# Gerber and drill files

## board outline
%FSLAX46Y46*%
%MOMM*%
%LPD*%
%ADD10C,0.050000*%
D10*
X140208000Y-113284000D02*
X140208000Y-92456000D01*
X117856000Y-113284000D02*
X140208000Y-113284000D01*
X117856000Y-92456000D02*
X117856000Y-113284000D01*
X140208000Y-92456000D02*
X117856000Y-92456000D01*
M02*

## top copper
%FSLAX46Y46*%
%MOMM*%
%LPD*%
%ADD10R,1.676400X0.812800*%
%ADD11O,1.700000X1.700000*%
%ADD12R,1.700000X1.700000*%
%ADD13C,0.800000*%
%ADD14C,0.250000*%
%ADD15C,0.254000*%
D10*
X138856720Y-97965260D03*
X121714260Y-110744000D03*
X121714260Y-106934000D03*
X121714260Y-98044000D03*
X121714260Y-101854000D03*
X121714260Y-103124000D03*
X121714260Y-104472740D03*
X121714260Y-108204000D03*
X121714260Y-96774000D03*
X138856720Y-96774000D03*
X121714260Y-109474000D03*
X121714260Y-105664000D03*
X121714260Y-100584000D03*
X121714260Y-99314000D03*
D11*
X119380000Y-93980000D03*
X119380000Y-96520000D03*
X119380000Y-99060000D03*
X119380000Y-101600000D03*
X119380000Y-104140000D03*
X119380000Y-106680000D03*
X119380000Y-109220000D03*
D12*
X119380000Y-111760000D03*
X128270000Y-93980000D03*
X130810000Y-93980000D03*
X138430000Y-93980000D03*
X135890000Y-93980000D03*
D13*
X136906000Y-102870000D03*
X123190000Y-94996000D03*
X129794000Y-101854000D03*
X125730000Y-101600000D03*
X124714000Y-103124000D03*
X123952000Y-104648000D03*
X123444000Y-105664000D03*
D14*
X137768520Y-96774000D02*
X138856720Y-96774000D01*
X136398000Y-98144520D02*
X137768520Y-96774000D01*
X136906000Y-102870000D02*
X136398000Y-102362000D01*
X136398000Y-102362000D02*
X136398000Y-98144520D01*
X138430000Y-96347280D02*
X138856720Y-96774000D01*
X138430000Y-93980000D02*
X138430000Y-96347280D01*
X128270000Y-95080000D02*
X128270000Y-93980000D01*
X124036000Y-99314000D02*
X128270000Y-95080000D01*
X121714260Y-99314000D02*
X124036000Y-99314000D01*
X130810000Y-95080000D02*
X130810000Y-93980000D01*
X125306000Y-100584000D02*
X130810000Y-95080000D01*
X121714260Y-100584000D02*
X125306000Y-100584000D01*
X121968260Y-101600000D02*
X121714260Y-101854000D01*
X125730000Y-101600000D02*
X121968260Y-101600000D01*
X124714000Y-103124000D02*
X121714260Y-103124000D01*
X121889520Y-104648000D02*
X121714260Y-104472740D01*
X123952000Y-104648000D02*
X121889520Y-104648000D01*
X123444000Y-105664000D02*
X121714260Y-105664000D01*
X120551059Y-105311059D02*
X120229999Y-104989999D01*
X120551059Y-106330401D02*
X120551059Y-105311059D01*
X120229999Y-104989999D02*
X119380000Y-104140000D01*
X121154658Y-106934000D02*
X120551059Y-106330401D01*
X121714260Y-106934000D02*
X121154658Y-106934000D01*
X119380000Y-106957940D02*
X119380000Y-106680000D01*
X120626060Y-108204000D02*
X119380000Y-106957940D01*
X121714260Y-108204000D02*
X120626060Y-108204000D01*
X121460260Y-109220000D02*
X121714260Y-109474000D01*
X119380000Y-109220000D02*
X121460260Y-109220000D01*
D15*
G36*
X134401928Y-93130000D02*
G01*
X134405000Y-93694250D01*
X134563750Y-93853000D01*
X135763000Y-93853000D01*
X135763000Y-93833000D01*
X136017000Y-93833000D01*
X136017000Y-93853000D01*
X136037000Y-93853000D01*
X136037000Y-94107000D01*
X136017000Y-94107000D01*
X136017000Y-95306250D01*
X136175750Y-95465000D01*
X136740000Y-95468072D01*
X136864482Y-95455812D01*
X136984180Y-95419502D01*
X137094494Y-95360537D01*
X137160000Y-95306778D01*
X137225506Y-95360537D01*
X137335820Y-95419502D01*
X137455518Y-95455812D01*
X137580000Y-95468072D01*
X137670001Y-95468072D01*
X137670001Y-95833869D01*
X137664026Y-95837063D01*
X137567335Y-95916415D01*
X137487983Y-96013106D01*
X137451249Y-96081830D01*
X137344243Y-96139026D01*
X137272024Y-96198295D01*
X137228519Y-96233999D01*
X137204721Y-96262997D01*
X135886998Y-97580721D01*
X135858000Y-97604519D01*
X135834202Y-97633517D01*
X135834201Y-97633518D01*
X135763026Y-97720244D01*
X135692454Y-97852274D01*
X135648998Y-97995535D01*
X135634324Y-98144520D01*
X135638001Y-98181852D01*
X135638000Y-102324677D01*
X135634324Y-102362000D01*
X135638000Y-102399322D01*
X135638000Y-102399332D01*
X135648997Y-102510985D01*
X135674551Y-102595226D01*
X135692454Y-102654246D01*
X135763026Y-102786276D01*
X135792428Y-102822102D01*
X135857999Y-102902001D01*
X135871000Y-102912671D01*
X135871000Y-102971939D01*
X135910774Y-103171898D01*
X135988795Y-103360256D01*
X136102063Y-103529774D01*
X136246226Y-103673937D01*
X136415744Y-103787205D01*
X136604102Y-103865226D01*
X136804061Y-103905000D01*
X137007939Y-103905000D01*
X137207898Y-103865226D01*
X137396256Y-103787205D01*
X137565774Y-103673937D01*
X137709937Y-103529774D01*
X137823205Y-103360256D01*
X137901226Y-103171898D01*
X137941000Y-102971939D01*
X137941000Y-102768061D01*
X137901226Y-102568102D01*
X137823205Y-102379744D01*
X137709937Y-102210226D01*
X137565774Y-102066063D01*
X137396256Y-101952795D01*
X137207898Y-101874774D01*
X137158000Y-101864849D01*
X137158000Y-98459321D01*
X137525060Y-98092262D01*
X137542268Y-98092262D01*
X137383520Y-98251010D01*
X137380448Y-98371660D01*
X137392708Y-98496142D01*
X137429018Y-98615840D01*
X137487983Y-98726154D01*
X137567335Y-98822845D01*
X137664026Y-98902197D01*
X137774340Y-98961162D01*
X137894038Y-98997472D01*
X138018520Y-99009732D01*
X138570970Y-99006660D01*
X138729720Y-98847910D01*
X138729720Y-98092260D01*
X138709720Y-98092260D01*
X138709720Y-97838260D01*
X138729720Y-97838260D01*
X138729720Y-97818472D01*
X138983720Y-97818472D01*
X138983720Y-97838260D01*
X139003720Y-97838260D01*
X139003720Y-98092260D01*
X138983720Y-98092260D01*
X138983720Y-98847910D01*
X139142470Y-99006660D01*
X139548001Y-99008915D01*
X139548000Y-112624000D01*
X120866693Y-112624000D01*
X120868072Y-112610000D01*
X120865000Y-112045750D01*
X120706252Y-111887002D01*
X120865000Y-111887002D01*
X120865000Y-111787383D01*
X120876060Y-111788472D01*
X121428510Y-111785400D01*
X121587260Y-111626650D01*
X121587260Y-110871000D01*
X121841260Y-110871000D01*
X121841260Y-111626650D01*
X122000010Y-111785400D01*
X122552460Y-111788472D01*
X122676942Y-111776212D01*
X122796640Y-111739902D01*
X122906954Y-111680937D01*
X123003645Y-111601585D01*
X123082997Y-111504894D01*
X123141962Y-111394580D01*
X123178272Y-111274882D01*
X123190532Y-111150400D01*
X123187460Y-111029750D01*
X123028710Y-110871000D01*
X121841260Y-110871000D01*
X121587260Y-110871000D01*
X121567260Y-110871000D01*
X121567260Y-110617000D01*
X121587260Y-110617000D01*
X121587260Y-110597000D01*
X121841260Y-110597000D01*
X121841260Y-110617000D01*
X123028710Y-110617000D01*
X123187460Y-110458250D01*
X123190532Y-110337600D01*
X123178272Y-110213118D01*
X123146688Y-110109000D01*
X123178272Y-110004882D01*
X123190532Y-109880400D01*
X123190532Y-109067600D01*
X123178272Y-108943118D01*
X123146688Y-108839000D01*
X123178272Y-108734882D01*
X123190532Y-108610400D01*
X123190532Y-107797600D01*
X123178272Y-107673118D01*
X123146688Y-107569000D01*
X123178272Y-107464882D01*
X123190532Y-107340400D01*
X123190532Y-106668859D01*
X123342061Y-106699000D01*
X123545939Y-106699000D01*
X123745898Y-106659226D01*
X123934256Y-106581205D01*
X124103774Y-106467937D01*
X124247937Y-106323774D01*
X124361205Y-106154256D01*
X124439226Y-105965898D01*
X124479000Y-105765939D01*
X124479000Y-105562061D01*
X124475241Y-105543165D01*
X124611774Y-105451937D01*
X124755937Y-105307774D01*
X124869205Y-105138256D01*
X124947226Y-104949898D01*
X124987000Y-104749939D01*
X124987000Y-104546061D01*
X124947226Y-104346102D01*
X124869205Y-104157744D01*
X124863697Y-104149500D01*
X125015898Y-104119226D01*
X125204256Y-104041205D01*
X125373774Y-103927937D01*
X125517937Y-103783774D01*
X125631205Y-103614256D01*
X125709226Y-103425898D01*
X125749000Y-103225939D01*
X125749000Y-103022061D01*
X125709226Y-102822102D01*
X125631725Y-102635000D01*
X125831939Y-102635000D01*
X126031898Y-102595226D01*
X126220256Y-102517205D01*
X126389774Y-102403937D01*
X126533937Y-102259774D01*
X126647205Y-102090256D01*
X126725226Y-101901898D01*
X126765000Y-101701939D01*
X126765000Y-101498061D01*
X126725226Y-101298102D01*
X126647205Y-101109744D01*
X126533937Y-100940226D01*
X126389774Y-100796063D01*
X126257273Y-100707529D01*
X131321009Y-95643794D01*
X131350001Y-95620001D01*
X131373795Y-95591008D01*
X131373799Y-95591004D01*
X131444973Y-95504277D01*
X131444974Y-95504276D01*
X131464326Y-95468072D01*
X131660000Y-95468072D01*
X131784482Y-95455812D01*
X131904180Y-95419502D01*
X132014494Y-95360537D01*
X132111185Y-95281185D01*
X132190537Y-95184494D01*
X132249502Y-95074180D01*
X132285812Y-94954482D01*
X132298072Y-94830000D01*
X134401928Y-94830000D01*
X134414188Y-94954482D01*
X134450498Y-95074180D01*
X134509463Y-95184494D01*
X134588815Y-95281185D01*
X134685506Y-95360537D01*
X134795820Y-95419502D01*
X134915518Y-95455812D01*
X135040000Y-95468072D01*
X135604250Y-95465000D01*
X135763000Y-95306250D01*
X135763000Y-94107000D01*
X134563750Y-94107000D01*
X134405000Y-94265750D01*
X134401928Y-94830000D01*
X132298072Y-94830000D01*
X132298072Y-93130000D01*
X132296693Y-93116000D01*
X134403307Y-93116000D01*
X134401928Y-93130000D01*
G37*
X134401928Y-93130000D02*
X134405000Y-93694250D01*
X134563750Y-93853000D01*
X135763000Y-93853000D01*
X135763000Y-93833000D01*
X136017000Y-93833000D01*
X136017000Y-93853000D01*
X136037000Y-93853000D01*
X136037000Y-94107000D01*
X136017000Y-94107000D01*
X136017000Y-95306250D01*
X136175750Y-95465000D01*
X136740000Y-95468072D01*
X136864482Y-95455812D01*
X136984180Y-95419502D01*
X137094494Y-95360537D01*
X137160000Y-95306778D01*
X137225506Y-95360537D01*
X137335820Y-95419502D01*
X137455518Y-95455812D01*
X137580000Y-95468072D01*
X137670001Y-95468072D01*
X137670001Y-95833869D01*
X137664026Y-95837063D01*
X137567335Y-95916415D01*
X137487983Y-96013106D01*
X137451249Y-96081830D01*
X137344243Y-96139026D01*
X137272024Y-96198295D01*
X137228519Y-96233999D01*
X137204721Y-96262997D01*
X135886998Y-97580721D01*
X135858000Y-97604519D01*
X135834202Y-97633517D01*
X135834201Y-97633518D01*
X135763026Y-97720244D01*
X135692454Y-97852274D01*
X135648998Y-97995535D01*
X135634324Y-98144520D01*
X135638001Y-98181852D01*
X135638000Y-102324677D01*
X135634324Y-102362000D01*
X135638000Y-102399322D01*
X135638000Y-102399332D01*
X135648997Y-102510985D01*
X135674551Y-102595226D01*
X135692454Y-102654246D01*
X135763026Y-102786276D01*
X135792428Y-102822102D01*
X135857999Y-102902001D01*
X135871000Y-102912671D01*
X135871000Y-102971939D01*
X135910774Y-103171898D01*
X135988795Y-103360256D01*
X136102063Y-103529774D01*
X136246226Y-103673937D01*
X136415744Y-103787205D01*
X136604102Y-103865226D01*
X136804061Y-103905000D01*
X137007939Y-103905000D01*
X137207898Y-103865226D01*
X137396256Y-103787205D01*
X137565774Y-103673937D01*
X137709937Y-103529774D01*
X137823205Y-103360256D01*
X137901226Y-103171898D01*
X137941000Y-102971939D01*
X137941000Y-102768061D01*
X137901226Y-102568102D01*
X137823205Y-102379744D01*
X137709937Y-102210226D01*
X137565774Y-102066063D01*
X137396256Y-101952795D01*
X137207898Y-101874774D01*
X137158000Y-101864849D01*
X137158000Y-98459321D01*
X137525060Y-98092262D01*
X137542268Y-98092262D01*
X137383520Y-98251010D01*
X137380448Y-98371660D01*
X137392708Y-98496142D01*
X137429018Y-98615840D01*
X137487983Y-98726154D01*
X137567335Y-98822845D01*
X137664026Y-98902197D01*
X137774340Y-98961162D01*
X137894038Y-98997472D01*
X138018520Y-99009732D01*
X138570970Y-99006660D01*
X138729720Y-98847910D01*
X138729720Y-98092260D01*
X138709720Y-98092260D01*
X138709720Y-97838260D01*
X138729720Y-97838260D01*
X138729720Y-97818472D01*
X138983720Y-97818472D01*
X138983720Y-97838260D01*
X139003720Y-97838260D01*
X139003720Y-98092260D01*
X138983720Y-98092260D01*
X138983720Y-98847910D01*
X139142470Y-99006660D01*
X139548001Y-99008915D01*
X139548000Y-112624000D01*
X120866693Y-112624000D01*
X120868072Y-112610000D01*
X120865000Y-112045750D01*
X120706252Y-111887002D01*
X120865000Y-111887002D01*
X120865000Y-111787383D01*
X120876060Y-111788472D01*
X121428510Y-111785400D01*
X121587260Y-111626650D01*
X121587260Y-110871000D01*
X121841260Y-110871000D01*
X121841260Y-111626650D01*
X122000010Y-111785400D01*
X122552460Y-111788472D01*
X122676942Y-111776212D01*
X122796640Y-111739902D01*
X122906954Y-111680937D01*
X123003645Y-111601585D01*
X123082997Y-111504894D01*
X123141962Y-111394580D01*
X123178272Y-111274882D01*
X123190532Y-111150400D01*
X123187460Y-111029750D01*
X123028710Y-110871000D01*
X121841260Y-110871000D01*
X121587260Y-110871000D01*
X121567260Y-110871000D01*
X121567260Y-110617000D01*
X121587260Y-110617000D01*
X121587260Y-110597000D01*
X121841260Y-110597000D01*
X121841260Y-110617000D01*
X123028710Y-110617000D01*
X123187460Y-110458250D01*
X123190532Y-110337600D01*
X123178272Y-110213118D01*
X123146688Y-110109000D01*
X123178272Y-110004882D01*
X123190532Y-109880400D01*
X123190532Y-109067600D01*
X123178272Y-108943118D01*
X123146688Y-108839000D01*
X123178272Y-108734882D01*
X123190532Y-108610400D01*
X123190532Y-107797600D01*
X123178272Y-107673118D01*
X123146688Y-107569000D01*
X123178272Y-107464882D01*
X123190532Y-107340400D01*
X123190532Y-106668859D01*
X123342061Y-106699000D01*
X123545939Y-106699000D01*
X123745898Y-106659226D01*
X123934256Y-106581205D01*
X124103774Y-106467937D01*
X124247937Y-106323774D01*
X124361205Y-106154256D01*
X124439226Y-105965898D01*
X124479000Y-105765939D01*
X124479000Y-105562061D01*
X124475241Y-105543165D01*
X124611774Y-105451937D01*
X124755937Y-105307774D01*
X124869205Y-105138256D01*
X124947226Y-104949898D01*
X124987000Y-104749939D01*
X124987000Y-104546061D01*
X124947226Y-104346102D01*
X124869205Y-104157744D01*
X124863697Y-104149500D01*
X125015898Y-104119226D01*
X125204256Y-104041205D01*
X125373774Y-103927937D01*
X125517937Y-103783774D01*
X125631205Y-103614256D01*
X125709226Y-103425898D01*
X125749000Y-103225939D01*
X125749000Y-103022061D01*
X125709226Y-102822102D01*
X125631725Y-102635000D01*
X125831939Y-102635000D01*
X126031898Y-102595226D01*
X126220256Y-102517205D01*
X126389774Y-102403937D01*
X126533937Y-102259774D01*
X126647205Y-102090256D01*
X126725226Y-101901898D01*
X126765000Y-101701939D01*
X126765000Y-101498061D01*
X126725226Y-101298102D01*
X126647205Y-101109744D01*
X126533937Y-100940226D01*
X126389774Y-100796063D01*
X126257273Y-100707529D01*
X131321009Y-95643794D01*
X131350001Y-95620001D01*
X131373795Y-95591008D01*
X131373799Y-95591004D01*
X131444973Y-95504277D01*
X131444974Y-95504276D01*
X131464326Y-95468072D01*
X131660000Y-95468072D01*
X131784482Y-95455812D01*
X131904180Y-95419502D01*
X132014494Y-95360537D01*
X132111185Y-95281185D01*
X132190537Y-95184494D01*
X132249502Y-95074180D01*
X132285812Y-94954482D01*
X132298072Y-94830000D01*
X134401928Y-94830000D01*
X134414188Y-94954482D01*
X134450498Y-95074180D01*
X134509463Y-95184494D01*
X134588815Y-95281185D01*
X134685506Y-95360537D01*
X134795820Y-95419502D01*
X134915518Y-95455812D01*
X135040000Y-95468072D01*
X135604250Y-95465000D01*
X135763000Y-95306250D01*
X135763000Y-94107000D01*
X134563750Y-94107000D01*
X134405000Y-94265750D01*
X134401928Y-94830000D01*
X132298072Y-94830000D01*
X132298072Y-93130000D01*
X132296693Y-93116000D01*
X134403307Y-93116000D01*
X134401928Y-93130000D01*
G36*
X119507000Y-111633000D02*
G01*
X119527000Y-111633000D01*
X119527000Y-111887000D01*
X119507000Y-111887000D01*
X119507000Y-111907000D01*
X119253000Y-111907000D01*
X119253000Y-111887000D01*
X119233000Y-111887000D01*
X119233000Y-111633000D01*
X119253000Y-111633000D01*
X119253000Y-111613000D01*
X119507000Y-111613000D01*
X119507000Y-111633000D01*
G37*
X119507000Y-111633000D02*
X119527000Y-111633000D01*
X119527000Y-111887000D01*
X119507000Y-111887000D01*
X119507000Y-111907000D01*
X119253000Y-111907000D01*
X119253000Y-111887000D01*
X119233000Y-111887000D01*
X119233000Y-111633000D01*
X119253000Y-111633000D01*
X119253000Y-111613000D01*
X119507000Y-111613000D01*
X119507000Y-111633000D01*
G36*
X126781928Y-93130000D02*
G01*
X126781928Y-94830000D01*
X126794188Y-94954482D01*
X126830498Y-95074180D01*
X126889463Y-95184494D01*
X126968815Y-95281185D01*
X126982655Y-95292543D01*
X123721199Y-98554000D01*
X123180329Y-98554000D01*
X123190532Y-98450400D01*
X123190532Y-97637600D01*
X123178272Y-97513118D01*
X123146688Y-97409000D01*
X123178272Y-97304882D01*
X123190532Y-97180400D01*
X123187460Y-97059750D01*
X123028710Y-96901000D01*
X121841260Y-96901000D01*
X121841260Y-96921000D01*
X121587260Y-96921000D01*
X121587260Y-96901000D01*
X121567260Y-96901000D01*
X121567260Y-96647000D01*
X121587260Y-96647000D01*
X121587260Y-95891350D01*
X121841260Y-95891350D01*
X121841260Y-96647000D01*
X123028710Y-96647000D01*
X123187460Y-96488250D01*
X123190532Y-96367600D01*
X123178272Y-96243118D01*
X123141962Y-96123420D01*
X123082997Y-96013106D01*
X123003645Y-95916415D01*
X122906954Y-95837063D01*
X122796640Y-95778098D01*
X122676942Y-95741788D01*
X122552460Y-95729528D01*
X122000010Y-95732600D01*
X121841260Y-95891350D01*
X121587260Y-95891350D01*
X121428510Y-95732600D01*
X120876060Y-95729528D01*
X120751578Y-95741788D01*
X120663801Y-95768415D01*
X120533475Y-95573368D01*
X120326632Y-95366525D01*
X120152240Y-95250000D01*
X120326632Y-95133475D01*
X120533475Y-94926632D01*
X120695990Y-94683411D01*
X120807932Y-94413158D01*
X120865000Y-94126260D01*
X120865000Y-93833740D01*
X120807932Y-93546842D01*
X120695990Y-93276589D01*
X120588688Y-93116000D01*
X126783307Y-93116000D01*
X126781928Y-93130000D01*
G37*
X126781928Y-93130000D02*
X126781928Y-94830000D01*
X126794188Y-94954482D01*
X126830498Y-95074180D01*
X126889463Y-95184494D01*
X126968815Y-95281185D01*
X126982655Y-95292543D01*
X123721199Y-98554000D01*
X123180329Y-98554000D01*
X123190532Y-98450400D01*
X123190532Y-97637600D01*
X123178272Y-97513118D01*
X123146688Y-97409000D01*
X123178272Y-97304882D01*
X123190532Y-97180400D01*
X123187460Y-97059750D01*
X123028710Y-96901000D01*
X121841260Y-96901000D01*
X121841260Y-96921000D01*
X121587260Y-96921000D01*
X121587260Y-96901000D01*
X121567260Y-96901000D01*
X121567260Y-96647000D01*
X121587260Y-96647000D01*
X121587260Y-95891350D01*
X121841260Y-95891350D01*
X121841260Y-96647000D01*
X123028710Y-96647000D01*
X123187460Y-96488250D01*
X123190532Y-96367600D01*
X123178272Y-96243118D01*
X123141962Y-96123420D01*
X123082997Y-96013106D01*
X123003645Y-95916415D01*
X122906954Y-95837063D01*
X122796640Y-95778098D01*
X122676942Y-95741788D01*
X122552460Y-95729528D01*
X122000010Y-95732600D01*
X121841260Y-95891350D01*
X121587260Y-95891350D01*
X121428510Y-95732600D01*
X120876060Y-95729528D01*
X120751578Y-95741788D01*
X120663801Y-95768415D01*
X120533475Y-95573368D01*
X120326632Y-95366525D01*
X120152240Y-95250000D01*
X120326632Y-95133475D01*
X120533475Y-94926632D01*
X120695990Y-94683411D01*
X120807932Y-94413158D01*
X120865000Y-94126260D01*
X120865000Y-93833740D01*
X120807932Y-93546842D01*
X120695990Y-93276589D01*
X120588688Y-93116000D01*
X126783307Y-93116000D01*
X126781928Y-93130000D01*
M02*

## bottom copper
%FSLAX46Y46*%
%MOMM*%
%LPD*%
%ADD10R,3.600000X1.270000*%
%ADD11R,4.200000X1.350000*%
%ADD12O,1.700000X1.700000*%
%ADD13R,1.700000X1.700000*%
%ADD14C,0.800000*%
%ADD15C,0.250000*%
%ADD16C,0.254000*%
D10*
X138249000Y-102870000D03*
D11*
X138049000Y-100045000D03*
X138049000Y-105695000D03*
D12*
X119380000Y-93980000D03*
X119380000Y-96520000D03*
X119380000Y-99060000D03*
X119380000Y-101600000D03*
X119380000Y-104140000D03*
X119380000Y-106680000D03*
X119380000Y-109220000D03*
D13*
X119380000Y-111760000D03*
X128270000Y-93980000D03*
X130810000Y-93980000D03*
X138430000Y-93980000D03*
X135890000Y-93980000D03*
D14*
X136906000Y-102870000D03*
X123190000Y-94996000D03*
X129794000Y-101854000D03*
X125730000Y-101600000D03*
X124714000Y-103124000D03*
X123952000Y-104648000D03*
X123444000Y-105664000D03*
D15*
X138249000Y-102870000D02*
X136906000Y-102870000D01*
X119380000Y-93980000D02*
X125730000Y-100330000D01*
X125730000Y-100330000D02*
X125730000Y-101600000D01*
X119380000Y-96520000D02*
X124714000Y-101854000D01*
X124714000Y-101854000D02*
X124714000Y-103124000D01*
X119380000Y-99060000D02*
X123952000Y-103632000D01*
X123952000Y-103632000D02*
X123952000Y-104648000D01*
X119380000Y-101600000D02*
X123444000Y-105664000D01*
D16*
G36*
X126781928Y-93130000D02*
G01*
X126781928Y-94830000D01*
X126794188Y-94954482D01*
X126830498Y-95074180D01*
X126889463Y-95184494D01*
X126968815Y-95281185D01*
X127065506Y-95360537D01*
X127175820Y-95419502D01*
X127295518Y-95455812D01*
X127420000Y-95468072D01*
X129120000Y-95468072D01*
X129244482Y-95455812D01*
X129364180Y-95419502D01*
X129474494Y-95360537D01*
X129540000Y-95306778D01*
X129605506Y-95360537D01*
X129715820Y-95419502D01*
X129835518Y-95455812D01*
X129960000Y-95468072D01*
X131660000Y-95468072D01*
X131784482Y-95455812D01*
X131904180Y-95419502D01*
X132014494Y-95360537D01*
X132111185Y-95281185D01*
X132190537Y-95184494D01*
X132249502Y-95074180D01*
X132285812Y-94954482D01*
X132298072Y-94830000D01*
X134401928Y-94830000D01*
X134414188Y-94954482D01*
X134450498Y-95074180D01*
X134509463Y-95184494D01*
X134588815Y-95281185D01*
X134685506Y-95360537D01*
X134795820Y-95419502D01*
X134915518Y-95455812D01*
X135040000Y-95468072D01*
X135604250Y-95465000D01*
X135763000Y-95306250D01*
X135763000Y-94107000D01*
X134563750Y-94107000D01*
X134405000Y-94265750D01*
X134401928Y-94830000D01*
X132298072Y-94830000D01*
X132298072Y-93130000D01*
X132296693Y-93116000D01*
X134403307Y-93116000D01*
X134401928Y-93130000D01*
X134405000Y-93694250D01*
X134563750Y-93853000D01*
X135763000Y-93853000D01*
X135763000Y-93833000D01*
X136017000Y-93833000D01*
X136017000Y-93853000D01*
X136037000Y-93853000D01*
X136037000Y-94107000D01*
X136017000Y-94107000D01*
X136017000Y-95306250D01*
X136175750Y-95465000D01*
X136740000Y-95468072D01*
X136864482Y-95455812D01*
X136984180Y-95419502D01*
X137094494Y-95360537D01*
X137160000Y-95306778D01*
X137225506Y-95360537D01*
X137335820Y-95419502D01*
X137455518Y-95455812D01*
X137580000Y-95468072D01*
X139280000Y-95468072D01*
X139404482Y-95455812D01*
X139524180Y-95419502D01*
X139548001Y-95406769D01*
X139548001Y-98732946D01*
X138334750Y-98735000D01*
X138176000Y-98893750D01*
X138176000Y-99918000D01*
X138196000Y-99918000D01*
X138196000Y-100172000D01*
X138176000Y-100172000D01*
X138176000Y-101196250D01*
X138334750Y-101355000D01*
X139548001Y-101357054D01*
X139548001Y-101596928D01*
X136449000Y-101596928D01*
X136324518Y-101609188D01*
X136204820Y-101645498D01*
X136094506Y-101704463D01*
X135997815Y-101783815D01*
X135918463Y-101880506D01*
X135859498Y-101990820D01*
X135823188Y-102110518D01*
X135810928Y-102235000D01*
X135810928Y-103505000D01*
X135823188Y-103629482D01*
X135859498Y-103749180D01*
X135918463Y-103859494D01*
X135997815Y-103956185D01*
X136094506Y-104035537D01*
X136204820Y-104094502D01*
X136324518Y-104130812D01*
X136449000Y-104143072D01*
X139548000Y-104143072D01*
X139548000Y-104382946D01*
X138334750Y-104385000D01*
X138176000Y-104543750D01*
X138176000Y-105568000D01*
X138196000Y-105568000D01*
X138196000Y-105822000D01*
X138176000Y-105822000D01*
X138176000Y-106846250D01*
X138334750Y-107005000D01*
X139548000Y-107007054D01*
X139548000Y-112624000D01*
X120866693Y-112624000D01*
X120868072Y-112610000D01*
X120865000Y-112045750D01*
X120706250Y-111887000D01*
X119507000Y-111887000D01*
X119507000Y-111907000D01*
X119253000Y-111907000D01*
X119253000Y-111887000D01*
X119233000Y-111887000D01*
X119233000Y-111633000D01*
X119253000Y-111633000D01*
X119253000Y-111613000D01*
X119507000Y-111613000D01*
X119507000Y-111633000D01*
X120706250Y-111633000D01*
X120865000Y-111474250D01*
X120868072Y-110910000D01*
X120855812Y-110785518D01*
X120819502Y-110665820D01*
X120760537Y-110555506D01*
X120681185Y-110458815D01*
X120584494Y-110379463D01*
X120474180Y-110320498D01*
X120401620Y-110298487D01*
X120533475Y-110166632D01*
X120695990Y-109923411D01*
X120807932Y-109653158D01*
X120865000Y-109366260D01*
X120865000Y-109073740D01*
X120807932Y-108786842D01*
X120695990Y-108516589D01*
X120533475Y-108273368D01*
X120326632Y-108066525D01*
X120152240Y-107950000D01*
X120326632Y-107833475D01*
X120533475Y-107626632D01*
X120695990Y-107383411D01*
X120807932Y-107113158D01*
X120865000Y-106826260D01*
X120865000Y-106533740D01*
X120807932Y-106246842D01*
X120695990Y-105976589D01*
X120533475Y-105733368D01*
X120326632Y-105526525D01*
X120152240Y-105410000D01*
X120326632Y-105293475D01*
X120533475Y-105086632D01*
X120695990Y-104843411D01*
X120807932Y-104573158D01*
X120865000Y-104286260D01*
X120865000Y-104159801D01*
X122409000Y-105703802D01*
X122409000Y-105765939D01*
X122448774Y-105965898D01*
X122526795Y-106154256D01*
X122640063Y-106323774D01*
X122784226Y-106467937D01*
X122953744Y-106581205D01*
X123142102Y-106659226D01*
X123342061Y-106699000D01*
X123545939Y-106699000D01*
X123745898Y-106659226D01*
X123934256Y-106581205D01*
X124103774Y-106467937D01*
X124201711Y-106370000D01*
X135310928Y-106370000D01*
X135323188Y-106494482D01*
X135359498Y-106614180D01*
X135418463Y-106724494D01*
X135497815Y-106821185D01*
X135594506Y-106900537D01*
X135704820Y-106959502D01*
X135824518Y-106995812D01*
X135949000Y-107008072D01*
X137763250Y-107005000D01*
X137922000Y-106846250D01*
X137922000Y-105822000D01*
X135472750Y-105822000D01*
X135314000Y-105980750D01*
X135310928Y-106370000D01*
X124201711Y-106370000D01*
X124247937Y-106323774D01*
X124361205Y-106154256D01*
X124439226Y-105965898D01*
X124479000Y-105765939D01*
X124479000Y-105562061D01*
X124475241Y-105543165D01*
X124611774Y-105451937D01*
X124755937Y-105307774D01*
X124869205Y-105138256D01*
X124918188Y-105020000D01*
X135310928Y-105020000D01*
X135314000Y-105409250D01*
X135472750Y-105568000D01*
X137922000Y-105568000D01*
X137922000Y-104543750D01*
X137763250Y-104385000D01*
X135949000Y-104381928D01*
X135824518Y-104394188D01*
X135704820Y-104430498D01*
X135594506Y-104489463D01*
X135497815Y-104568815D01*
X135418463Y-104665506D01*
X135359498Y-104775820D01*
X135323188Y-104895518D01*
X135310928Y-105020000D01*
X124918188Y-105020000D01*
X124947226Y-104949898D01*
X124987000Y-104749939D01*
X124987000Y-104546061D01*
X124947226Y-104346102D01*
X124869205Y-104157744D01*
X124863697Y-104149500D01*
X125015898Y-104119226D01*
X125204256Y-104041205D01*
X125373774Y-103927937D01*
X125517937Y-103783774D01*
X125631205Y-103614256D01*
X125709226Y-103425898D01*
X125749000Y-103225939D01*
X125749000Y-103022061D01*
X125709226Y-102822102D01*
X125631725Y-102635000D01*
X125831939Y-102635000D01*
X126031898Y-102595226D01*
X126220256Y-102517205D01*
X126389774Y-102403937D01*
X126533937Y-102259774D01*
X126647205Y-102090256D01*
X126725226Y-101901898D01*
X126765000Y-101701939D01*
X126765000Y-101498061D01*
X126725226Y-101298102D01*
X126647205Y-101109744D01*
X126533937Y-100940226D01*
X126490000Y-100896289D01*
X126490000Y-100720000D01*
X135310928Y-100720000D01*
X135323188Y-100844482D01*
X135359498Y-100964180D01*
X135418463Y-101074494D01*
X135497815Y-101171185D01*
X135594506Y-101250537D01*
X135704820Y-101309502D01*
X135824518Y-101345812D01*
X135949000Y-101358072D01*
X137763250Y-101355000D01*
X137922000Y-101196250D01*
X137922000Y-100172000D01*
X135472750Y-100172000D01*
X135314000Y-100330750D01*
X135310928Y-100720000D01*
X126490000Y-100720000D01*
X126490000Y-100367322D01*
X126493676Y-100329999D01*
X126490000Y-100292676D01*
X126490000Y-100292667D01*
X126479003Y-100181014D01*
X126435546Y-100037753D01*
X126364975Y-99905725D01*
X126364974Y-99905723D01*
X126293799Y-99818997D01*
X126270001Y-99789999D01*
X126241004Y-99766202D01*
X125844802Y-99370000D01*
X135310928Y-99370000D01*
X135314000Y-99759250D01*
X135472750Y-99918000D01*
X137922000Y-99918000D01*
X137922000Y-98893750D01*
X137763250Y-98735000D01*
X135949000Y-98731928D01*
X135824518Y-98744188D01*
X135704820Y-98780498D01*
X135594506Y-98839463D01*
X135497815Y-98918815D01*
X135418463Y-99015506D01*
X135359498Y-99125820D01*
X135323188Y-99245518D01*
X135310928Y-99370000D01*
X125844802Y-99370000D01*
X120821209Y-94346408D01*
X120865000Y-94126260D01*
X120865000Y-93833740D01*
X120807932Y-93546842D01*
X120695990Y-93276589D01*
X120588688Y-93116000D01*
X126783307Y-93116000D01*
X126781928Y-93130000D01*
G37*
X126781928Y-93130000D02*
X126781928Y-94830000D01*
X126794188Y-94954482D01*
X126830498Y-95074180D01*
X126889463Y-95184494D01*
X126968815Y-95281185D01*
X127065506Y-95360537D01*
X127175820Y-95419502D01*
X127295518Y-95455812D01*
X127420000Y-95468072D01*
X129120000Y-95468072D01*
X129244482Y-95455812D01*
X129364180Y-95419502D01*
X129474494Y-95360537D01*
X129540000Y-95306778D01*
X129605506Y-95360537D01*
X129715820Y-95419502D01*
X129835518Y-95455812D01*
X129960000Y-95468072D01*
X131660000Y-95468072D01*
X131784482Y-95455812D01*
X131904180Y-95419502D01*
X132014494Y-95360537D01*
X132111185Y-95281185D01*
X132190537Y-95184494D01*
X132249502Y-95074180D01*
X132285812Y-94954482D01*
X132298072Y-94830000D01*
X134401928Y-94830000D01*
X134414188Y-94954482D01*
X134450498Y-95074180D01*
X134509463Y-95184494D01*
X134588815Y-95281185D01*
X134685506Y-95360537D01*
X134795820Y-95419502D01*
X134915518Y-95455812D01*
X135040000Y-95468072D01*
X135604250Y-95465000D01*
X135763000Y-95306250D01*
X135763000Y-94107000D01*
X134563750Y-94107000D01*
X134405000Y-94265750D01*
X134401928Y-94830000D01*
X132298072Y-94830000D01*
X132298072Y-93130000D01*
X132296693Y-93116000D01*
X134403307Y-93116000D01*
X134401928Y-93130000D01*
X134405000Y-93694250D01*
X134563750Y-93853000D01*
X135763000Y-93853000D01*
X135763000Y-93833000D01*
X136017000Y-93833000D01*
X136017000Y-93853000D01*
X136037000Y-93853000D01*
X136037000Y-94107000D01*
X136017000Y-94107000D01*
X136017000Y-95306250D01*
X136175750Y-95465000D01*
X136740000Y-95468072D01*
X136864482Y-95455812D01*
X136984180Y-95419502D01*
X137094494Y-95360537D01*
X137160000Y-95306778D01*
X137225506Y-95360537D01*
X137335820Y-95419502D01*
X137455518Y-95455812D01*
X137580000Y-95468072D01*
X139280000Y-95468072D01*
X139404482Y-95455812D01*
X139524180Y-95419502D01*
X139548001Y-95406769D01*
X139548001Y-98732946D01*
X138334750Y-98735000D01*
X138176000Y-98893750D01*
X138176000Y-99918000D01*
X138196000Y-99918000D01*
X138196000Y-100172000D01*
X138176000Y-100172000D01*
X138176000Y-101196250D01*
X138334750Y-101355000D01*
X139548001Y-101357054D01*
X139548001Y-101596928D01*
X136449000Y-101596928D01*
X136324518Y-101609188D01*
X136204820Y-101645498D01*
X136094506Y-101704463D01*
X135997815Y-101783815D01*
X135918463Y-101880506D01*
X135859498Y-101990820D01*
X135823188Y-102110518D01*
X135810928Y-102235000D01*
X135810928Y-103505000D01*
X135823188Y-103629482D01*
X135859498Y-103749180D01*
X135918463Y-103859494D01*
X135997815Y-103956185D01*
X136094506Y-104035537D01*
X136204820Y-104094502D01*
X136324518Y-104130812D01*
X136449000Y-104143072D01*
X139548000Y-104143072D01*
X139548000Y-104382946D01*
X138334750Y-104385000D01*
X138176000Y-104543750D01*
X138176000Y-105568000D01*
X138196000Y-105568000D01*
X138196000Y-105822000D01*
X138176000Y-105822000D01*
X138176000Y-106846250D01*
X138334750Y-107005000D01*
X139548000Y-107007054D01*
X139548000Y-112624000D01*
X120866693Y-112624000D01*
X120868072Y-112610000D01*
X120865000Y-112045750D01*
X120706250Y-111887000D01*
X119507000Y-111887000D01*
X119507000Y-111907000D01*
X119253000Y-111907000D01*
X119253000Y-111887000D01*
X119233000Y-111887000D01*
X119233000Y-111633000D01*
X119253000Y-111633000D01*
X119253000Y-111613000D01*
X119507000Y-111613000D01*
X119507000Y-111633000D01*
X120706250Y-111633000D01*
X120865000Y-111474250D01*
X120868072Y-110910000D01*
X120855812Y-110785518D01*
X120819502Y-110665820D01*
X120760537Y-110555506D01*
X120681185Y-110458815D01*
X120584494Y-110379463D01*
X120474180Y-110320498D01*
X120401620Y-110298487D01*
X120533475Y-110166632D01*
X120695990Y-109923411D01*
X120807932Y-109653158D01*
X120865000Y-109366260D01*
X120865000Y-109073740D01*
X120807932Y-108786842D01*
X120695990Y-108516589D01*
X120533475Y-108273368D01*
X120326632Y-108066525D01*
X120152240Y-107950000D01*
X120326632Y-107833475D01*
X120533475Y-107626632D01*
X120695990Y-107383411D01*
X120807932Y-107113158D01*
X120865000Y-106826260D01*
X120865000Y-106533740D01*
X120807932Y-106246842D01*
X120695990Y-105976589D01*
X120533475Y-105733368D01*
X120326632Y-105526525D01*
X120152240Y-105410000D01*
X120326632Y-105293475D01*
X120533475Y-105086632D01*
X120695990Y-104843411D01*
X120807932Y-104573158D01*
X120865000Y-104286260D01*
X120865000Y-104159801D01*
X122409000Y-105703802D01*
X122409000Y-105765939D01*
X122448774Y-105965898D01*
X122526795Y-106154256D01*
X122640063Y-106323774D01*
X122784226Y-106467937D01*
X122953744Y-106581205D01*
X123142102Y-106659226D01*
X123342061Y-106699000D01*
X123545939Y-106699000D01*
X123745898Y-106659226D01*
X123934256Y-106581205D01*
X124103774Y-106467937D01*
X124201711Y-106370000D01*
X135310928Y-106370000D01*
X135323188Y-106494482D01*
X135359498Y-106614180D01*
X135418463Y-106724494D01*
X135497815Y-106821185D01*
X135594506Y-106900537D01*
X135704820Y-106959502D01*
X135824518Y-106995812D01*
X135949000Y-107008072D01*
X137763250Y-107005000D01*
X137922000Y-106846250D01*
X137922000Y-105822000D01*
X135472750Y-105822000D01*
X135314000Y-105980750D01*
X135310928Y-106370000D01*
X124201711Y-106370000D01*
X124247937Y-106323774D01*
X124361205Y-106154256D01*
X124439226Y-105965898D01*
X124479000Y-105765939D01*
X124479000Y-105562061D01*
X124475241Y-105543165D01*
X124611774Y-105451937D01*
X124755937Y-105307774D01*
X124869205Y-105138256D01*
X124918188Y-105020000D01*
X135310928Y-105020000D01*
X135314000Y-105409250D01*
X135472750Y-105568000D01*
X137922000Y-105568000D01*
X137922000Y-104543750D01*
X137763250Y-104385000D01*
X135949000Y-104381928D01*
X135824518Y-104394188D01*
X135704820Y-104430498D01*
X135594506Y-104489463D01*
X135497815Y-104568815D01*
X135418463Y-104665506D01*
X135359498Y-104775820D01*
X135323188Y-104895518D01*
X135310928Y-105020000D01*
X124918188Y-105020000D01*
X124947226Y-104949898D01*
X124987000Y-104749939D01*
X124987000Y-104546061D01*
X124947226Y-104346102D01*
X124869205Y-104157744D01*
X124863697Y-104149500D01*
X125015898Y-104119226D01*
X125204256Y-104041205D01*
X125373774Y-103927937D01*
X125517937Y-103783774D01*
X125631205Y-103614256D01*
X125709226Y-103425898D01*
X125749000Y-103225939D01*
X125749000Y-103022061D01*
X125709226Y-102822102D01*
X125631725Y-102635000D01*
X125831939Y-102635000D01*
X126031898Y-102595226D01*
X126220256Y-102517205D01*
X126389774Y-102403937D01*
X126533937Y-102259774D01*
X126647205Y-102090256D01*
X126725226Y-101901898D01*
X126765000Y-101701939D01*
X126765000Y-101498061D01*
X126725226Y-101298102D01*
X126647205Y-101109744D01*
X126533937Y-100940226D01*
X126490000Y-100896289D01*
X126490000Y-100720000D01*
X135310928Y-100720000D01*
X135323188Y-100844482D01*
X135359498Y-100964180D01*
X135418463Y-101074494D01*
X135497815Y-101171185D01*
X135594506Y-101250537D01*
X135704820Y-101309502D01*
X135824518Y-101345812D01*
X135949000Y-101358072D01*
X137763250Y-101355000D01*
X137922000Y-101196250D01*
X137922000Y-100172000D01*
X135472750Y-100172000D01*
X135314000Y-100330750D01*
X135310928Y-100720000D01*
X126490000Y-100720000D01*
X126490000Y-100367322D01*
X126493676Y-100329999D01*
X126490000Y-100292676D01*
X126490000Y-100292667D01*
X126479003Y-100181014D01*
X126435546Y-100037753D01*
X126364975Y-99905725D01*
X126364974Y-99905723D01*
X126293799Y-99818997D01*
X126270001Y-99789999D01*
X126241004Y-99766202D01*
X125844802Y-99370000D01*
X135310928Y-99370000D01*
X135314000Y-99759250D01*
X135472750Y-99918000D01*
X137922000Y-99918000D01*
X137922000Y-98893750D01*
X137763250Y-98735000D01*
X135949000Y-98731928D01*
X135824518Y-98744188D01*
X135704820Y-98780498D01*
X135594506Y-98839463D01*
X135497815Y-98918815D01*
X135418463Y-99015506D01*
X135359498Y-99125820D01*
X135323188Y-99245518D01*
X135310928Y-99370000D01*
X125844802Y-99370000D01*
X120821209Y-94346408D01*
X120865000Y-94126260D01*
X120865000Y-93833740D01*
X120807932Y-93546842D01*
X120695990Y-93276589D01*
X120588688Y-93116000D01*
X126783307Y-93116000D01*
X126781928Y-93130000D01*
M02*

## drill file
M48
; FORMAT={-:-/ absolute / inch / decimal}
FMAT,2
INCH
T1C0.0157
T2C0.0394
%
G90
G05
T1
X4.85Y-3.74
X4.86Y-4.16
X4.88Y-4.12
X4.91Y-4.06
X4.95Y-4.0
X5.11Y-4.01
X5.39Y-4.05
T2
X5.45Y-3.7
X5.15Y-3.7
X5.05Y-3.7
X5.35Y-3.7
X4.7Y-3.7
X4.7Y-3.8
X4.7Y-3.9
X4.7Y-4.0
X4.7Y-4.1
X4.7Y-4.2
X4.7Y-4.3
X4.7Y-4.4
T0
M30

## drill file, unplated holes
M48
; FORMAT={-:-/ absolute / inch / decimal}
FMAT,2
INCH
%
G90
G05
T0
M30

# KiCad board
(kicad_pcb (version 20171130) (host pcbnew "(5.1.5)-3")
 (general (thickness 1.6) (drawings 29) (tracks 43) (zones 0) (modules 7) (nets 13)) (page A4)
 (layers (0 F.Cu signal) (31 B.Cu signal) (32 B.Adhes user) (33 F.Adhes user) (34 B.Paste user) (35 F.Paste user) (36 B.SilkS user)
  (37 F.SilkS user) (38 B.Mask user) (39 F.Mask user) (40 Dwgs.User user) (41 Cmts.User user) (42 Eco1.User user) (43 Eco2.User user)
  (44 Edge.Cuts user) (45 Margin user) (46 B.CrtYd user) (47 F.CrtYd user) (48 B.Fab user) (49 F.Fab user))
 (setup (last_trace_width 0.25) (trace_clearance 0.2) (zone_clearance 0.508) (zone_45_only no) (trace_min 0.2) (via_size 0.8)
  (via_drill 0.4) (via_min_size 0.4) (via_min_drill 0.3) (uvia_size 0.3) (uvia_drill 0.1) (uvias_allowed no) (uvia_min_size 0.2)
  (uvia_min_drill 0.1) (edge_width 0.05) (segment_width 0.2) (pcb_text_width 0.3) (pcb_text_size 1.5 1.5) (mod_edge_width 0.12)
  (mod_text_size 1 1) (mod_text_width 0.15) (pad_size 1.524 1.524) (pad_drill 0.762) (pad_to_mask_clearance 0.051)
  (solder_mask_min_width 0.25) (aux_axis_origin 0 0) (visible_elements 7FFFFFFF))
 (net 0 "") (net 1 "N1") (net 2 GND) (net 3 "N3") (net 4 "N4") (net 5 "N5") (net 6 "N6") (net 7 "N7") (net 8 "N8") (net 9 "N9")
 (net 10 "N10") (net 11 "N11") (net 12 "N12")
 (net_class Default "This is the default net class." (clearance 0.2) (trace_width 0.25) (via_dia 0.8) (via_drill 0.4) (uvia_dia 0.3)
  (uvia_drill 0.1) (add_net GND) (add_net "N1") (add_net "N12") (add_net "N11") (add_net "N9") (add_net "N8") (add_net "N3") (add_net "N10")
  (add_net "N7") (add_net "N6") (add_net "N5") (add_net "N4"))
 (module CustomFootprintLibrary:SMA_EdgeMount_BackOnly (layer F.Cu) (at 138.049 102.87 90)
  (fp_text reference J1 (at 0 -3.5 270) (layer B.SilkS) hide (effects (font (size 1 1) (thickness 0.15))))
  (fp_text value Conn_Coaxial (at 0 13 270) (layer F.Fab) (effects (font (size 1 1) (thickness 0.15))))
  (pad 1 smd rect (at 0 0.2 90) (size 1.27 3.6) (layers B.Cu B.Paste B.Mask) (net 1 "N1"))
  (pad 2 smd rect (at 2.825 0 90) (size 1.35 4.2) (layers B.Cu B.Paste B.Mask) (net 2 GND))
  (pad 2 smd rect (at -2.825 0 90) (size 1.35 4.2) (layers B.Cu B.Paste B.Mask) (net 2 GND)))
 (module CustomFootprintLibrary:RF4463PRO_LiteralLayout (layer F.Cu) (at 130.302 103.378)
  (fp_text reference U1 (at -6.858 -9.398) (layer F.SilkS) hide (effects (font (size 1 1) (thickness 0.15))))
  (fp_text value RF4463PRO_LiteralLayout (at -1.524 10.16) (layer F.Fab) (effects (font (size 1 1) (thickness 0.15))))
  (pad 13 smd rect (at 8.55472 -5.41274) (size 1.6764 0.8128) (layers F.Cu F.Paste F.Mask) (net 2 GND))
  (pad 12 smd rect (at -8.58774 7.366) (size 1.6764 0.8128) (layers F.Cu F.Paste F.Mask) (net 2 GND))
  (pad 9 smd rect (at -8.58774 3.556) (size 1.6764 0.8128) (layers F.Cu F.Paste F.Mask) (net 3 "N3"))
  (pad 2 smd rect (at -8.58774 -5.334) (size 1.6764 0.8128) (layers F.Cu F.Paste F.Mask) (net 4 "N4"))
  (pad 5 smd rect (at -8.58774 -1.524) (size 1.6764 0.8128) (layers F.Cu F.Paste F.Mask) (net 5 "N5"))
  (pad 6 smd rect (at -8.58774 -0.254) (size 1.6764 0.8128) (layers F.Cu F.Paste F.Mask) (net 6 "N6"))
  (pad 7 smd rect (at -8.58774 1.09474) (size 1.6764 0.8128) (layers F.Cu F.Paste F.Mask) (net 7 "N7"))
  (pad 10 smd rect (at -8.58774 4.826) (size 1.6764 0.8128) (layers F.Cu F.Paste F.Mask) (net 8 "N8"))
  (pad 1 smd rect (at -8.58774 -6.604) (size 1.6764 0.8128) (layers F.Cu F.Paste F.Mask) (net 2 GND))
  (pad 14 smd rect (at 8.55472 -6.604) (size 1.6764 0.8128) (layers F.Cu F.Paste F.Mask) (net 1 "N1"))
  (pad 11 smd rect (at -8.58774 6.096) (size 1.6764 0.8128) (layers F.Cu F.Paste F.Mask) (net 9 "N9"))
  (pad 8 smd rect (at -8.58774 2.286) (size 1.6764 0.8128) (layers F.Cu F.Paste F.Mask) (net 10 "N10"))
  (pad 4 smd rect (at -8.58774 -2.794) (size 1.6764 0.8128) (layers F.Cu F.Paste F.Mask) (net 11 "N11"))
  (pad 3 smd rect (at -8.58774 -4.064) (size 1.6764 0.8128) (layers F.Cu F.Paste F.Mask) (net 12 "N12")))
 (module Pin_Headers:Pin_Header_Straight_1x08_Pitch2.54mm (layer F.Cu) (at 119.38 111.76 180)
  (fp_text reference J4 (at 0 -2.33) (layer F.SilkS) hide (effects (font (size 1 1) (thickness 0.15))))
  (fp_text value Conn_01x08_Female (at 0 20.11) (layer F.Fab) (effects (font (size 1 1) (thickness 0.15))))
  (pad 8 thru_hole oval (at 0 17.78 180) (size 1.7 1.7) (drill 1) (layers *.Cu *.Mask) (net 5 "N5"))
  (pad 7 thru_hole oval (at 0 15.24 180) (size 1.7 1.7) (drill 1) (layers *.Cu *.Mask) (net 6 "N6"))
  (pad 6 thru_hole oval (at 0 12.7 180) (size 1.7 1.7) (drill 1) (layers *.Cu *.Mask) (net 7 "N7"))
  (pad 5 thru_hole oval (at 0 10.16 180) (size 1.7 1.7) (drill 1) (layers *.Cu *.Mask) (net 10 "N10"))
  (pad 4 thru_hole oval (at 0 7.62 180) (size 1.7 1.7) (drill 1) (layers *.Cu *.Mask) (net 3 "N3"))
  (pad 3 thru_hole oval (at 0 5.08 180) (size 1.7 1.7) (drill 1) (layers *.Cu *.Mask) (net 8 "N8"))
  (pad 2 thru_hole oval (at 0 2.54 180) (size 1.7 1.7) (drill 1) (layers *.Cu *.Mask) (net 9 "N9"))
  (pad 1 thru_hole rect (at 0 0 180) (size 1.7 1.7) (drill 1) (layers *.Cu *.Mask) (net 2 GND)))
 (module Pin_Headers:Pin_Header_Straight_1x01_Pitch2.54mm (layer F.Cu) (at 128.27 93.98)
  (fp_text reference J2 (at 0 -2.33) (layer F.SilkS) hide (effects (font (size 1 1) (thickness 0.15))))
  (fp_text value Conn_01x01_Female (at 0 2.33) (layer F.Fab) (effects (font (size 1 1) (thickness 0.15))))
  (pad 1 thru_hole rect (at 0 0) (size 1.7 1.7) (drill 1) (layers *.Cu *.Mask) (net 12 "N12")))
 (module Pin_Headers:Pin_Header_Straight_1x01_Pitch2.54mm (layer F.Cu) (at 130.81 93.98)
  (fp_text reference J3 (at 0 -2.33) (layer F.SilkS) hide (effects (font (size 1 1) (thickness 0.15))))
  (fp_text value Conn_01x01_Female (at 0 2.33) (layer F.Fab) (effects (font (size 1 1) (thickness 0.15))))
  (pad 1 thru_hole rect (at 0 0) (size 1.7 1.7) (drill 1) (layers *.Cu *.Mask) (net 11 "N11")))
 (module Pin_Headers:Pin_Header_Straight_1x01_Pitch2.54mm (layer F.Cu) (at 138.43 93.98)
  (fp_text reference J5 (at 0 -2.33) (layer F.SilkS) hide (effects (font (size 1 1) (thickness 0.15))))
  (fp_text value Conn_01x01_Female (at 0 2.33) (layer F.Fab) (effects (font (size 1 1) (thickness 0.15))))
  (pad 1 thru_hole rect (at 0 0) (size 1.7 1.7) (drill 1) (layers *.Cu *.Mask) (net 1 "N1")))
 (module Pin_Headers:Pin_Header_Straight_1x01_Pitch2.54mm (layer F.Cu) (at 135.89 93.98)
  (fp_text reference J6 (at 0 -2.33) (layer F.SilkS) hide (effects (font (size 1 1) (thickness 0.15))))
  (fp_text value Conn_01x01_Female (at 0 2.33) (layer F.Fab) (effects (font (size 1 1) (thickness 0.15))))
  (pad 1 thru_hole rect (at 0 0) (size 1.7 1.7) (drill 1) (layers *.Cu *.Mask) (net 2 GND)))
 (gr_line (start 140.208 113.284) (end 140.208 92.456) (layer Edge.Cuts) (width 0.05))
 (gr_line (start 117.856 113.284) (end 140.208 113.284) (layer Edge.Cuts) (width 0.05))
 (gr_line (start 117.856 92.456) (end 117.856 113.284) (layer Edge.Cuts) (width 0.05))
 (gr_line (start 140.208 92.456) (end 117.856 92.456) (layer Edge.Cuts) (width 0.05))
 (via (at 136.906 102.87) (size 0.8) (drill 0.4) (layers F.Cu B.Cu) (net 1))
 (segment (start 138.249 102.87) (end 136.906 102.87) (width 0.25) (layer B.Cu) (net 1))
 (segment (start 137.76852 96.774) (end 138.85672 96.774) (width 0.25) (layer F.Cu) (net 1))
 (segment (start 136.398 98.14452) (end 137.76852 96.774) (width 0.25) (layer F.Cu) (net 1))
 (segment (start 136.906 102.87) (end 136.398 102.362) (width 0.25) (layer F.Cu) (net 1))
 (segment (start 136.398 102.362) (end 136.398 98.14452) (width 0.25) (layer F.Cu) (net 1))
 (segment (start 138.43 96.34728) (end 138.85672 96.774) (width 0.25) (layer F.Cu) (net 1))
 (segment (start 138.43 93.98) (end 138.43 96.34728) (width 0.25) (layer F.Cu) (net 1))
 (via (at 123.19 94.996) (size 0.8) (drill 0.4) (layers F.Cu B.Cu) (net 2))
 (via (at 129.794 101.854) (size 0.8) (drill 0.4) (layers F.Cu B.Cu) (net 2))
 (segment (start 128.27 95.08) (end 128.27 93.98) (width 0.25) (layer F.Cu) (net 12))
 (segment (start 124.036 99.314) (end 128.27 95.08) (width 0.25) (layer F.Cu) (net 12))
 (segment (start 121.71426 99.314) (end 124.036 99.314) (width 0.25) (layer F.Cu) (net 12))
 (segment (start 130.81 95.08) (end 130.81 93.98) (width 0.25) (layer F.Cu) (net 11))
 (segment (start 125.306 100.584) (end 130.81 95.08) (width 0.25) (layer F.Cu) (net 11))
 (segment (start 121.71426 100.584) (end 125.306 100.584) (width 0.25) (layer F.Cu) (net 11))
 (via (at 125.73 101.6) (size 0.8) (drill 0.4) (layers F.Cu B.Cu) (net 5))
 (segment (start 119.38 93.98) (end 125.73 100.33) (width 0.25) (layer B.Cu) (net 5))
 (segment (start 125.73 100.33) (end 125.73 101.6) (width 0.25) (layer B.Cu) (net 5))
 (segment (start 121.96826 101.6) (end 121.71426 101.854) (width 0.25) (layer F.Cu) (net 5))
 (segment (start 125.73 101.6) (end 121.96826 101.6) (width 0.25) (layer F.Cu) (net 5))
 (via (at 124.714 103.124) (size 0.8) (drill 0.4) (layers F.Cu B.Cu) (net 6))
 (segment (start 119.38 96.52) (end 124.714 101.854) (width 0.25) (layer B.Cu) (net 6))
 (segment (start 124.714 101.854) (end 124.714 103.124) (width 0.25) (layer B.Cu) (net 6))
 (segment (start 124.714 103.124) (end 121.71426 103.124) (width 0.25) (layer F.Cu) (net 6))
 (via (at 123.952 104.648) (size 0.8) (drill 0.4) (layers F.Cu B.Cu) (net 7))
 (segment (start 119.38 99.06) (end 123.952 103.632) (width 0.25) (layer B.Cu) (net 7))
 (segment (start 123.952 103.632) (end 123.952 104.648) (width 0.25) (layer B.Cu) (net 7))
 (segment (start 121.88952 104.648) (end 121.71426 104.47274) (width 0.25) (layer F.Cu) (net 7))
 (segment (start 123.952 104.648) (end 121.88952 104.648) (width 0.25) (layer F.Cu) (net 7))
 (via (at 123.444 105.664) (size 0.8) (drill 0.4) (layers F.Cu B.Cu) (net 10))
 (segment (start 119.38 101.6) (end 123.444 105.664) (width 0.25) (layer B.Cu) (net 10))
 (segment (start 123.444 105.664) (end 121.71426 105.664) (width 0.25) (layer F.Cu) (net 10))
 (segment (start 120.551059 105.311059) (end 120.229999 104.989999) (width 0.25) (layer F.Cu) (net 3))
 (segment (start 120.551059 106.330401) (end 120.551059 105.311059) (width 0.25) (layer F.Cu) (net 3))
 (segment (start 120.229999 104.989999) (end 119.38 104.14) (width 0.25) (layer F.Cu) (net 3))
 (segment (start 121.154658 106.934) (end 120.551059 106.330401) (width 0.25) (layer F.Cu) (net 3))
 (segment (start 121.71426 106.934) (end 121.154658 106.934) (width 0.25) (layer F.Cu) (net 3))
 (segment (start 119.38 106.95794) (end 119.38 106.68) (width 0.25) (layer F.Cu) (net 8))
 (segment (start 120.62606 108.204) (end 119.38 106.95794) (width 0.25) (layer F.Cu) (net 8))
 (segment (start 121.71426 108.204) (end 120.62606 108.204) (width 0.25) (layer F.Cu) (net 8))
 (segment (start 121.46026 109.22) (end 121.71426 109.474) (width 0.25) (layer F.Cu) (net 9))
 (segment (start 119.38 109.22) (end 121.46026 109.22) (width 0.25) (layer F.Cu) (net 9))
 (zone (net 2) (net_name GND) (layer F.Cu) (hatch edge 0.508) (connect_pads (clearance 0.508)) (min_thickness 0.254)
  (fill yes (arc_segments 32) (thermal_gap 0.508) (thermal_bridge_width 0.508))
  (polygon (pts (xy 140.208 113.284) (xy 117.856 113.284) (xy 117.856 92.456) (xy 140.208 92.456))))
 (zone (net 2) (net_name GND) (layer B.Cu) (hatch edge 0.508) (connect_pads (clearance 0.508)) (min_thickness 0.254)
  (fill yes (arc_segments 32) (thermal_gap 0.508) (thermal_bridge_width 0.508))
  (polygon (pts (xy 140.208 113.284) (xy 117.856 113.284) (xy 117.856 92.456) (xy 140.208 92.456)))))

